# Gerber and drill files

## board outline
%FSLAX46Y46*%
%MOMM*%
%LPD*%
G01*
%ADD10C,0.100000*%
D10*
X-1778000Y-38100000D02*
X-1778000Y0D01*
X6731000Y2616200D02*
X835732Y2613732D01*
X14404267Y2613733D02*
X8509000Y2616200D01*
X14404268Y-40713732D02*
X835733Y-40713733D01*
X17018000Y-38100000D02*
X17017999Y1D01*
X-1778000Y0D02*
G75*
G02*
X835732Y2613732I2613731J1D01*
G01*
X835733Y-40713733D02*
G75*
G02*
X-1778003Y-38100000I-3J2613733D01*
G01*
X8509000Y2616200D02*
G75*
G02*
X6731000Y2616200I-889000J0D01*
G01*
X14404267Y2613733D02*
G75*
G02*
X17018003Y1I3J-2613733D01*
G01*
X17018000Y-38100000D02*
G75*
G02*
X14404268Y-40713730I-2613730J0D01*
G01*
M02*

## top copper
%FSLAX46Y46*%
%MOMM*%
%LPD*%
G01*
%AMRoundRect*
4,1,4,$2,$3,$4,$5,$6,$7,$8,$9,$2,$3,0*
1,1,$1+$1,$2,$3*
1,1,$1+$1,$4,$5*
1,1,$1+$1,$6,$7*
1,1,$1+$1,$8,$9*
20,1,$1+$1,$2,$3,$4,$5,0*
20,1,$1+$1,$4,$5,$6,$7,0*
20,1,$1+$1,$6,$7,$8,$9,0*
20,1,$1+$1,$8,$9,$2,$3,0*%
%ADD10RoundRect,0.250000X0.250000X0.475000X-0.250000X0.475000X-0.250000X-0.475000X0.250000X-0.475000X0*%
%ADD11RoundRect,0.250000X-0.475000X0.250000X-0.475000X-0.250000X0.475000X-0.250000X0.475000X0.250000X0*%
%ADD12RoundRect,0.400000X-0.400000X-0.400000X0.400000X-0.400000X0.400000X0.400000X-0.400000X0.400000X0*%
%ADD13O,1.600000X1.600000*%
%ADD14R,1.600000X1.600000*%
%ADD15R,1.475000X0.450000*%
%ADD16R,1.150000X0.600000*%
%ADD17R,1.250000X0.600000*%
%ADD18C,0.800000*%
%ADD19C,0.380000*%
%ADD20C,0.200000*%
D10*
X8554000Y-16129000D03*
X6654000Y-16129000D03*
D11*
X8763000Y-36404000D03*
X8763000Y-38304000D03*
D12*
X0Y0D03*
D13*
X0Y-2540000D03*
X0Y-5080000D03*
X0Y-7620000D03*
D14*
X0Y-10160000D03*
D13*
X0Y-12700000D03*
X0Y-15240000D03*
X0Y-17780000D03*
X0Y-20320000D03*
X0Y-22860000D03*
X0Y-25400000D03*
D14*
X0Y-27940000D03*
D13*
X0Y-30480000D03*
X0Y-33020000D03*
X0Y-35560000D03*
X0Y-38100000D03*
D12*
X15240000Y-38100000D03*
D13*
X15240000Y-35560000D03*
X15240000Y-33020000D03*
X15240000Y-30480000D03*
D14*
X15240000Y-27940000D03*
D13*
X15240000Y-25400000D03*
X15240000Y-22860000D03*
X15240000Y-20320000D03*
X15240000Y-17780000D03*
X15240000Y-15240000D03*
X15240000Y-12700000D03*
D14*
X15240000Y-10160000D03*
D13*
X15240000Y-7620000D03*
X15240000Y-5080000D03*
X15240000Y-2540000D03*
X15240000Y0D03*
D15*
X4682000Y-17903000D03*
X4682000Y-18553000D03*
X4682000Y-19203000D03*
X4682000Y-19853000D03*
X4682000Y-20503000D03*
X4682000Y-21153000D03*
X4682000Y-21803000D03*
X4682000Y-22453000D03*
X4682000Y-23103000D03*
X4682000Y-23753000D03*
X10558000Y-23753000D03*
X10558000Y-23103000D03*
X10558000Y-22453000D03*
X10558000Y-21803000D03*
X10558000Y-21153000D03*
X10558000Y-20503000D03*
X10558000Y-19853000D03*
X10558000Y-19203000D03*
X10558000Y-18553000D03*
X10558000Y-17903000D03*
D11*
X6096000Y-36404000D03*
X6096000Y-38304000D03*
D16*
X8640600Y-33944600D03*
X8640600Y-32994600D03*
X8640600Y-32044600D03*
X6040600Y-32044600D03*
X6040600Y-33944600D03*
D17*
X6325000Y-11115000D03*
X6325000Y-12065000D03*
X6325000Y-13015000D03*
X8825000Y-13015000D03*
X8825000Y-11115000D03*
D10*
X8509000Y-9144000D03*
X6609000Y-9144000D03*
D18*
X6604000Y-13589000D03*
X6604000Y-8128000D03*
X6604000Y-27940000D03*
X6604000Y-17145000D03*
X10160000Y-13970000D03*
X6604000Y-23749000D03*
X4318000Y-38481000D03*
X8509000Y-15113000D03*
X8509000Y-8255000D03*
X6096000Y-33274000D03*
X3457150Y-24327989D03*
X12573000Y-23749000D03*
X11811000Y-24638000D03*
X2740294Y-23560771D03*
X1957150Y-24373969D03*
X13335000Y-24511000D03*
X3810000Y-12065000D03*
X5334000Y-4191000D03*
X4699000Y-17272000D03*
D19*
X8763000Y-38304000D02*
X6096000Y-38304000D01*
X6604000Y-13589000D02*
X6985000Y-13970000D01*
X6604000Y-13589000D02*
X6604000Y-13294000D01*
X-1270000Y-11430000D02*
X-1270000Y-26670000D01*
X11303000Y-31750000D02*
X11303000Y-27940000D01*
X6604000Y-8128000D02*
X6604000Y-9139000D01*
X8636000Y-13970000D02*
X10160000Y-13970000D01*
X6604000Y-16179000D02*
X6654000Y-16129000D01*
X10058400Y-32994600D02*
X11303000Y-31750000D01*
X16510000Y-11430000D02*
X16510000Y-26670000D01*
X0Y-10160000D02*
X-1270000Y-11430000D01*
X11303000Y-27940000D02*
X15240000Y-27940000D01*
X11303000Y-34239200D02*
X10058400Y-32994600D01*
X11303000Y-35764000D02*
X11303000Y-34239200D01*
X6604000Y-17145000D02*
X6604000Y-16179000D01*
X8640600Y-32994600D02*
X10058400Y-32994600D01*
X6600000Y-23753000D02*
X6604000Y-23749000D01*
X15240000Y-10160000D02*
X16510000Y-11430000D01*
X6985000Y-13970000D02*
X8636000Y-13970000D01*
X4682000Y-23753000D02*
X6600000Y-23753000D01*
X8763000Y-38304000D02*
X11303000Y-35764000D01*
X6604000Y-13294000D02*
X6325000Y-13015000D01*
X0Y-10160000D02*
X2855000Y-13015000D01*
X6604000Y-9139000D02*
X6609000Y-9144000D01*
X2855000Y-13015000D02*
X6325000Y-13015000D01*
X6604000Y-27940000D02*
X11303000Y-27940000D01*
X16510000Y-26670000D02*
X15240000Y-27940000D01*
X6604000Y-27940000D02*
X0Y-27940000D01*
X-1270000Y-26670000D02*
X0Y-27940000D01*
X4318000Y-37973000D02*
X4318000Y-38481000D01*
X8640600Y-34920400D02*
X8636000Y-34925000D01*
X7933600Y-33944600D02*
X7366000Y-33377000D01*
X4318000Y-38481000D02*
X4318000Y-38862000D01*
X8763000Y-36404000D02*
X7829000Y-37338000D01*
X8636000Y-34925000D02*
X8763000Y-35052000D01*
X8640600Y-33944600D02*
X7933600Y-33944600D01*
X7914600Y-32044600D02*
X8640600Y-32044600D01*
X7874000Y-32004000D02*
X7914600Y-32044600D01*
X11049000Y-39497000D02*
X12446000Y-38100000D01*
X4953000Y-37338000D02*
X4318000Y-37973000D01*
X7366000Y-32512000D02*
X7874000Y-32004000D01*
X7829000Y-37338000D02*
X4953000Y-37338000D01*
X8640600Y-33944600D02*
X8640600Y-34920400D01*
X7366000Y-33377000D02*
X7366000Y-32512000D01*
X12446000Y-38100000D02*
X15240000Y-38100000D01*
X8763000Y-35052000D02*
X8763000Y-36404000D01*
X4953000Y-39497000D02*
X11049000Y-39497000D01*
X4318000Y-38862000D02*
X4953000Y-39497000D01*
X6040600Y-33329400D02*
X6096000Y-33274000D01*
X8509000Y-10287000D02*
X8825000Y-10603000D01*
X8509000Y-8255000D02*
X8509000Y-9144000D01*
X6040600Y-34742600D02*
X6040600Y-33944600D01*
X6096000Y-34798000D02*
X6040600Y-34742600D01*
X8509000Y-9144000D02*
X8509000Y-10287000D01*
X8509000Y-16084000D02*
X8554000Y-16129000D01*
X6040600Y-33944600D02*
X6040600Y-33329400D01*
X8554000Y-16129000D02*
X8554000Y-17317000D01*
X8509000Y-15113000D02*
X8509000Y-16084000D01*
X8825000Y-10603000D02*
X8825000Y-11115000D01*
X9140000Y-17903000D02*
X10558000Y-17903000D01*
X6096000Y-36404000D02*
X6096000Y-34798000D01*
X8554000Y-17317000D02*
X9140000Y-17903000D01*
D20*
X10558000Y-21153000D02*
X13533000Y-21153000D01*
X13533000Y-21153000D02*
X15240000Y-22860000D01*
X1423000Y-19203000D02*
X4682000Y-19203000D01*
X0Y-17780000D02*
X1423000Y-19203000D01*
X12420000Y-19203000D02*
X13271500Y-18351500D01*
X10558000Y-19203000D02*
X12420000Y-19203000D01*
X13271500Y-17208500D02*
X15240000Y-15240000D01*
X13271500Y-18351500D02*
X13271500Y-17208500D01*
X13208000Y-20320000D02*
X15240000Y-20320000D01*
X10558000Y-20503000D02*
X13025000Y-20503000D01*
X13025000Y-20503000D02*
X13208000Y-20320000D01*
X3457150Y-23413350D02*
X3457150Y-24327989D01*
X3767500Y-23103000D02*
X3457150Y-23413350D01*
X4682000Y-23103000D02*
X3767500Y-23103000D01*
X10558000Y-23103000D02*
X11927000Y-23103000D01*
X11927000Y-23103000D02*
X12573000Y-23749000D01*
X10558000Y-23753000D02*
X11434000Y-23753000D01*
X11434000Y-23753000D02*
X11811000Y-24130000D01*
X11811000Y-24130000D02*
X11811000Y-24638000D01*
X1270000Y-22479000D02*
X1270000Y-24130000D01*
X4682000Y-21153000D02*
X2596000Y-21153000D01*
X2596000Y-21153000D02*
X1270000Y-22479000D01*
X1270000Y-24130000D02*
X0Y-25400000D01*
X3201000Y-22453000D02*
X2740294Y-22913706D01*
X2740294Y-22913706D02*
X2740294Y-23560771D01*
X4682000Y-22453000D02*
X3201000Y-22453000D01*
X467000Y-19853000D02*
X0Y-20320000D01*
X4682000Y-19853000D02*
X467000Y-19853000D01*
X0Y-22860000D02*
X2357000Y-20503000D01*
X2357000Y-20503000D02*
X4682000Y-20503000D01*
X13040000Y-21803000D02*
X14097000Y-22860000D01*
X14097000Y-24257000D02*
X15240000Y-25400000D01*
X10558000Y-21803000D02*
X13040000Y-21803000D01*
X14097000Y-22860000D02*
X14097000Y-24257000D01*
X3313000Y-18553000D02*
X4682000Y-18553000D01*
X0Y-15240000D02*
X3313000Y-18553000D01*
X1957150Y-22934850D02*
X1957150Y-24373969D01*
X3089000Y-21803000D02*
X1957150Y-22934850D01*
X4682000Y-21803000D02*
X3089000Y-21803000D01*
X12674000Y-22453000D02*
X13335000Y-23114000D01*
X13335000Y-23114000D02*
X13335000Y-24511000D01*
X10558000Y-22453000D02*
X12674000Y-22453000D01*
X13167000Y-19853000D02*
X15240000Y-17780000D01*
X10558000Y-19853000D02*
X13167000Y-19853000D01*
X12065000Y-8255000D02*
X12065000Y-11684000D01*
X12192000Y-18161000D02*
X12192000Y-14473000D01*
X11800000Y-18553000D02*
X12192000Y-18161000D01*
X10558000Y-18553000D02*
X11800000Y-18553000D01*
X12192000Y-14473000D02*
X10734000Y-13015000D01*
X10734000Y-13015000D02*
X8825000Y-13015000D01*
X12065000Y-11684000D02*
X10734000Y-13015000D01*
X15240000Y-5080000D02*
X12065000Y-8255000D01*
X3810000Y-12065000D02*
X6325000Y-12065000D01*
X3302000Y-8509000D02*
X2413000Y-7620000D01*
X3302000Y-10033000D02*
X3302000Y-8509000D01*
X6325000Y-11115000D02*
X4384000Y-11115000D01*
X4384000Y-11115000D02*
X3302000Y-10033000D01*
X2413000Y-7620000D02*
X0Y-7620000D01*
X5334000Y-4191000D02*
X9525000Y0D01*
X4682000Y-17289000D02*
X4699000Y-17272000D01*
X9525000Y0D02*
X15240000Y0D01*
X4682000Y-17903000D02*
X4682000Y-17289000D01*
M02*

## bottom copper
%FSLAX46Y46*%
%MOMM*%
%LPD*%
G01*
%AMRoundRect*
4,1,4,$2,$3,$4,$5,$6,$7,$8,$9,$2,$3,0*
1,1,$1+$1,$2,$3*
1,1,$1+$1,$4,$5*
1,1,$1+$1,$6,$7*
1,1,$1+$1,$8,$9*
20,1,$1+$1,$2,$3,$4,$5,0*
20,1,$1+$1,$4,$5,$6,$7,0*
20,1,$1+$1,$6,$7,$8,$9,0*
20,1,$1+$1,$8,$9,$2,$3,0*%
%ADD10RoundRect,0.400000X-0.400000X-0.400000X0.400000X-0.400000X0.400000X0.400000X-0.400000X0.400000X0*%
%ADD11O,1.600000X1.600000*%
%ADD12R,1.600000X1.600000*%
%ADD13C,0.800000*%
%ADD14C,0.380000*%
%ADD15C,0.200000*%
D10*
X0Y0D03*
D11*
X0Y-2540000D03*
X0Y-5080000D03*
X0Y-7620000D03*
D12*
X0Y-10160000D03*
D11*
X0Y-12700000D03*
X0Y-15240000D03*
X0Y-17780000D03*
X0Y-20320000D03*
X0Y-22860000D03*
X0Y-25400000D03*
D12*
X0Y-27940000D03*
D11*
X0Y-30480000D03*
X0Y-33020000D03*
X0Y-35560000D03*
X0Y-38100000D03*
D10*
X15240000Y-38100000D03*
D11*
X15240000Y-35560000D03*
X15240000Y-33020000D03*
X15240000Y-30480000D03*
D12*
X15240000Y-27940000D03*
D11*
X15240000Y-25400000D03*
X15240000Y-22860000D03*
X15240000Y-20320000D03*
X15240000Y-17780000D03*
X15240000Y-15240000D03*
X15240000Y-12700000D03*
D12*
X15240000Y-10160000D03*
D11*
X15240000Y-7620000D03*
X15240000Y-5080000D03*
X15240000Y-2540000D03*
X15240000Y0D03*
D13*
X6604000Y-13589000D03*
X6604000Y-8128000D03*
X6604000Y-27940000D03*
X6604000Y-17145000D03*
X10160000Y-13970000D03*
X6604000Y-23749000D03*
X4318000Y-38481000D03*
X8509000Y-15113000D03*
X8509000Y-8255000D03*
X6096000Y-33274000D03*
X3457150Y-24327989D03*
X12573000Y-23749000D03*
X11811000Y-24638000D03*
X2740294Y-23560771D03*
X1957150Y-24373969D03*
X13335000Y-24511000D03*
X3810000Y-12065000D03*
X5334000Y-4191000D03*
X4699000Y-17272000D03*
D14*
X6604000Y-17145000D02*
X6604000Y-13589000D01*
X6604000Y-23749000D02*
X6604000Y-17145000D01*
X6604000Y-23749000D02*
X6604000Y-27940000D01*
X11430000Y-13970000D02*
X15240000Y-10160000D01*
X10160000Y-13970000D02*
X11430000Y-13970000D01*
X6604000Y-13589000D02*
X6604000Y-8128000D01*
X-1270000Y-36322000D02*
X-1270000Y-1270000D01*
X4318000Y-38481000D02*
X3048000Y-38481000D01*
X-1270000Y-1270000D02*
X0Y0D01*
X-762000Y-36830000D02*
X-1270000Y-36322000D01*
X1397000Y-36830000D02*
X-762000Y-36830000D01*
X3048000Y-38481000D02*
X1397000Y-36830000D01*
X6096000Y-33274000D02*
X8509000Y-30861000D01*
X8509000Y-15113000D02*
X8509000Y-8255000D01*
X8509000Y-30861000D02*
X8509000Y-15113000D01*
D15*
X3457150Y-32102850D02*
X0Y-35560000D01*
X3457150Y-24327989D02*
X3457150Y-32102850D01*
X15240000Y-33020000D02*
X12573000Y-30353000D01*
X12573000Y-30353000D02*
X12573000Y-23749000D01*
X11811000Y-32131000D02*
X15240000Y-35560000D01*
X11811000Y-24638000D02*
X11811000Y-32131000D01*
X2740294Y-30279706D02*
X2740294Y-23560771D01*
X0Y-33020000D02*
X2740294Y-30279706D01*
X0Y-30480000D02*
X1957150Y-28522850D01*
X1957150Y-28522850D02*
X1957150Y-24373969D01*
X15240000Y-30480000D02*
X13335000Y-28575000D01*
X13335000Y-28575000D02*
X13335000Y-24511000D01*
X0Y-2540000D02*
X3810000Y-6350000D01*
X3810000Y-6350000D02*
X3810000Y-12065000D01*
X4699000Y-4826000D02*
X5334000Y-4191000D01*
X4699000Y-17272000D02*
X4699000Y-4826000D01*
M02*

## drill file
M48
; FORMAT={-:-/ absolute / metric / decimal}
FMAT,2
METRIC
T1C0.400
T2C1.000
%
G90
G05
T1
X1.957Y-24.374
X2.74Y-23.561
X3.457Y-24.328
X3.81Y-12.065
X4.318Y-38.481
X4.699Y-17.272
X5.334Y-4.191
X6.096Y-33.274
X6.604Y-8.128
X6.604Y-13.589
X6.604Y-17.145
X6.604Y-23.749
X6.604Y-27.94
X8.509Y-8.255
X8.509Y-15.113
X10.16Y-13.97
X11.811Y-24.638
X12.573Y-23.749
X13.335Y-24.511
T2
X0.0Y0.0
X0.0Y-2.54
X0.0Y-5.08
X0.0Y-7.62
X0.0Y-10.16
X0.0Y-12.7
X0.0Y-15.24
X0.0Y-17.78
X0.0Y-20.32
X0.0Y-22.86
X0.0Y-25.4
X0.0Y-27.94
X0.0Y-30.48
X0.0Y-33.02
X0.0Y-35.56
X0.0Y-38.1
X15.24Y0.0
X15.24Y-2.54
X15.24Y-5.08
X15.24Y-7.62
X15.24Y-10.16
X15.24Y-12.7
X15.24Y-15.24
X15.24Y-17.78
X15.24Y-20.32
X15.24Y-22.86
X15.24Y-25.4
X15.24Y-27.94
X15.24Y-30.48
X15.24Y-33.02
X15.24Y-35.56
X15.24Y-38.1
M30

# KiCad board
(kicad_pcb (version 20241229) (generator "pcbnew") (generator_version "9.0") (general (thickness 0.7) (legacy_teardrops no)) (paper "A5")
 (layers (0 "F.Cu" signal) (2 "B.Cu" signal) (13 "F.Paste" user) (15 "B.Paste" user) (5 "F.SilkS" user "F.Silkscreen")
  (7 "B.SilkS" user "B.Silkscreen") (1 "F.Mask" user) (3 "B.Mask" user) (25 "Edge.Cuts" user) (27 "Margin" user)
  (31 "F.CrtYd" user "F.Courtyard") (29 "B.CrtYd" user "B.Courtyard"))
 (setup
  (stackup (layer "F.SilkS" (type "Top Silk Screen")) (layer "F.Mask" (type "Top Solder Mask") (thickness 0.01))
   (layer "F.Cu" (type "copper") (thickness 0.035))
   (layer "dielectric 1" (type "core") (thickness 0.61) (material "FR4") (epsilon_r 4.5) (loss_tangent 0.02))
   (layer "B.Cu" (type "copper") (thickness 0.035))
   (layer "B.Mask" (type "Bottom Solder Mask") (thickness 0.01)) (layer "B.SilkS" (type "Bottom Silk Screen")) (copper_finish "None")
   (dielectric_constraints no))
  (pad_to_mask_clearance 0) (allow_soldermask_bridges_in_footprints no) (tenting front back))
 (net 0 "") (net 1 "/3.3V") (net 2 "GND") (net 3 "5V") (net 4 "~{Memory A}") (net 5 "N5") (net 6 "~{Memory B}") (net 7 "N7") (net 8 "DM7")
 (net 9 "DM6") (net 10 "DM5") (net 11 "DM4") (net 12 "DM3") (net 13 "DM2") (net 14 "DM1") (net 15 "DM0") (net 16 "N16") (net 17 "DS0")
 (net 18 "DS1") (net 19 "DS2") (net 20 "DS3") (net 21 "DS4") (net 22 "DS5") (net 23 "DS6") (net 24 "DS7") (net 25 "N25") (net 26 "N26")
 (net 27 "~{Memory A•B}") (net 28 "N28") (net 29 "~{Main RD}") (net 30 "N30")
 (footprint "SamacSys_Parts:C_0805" (layer "F.Cu") (at 7.62 16.129 90)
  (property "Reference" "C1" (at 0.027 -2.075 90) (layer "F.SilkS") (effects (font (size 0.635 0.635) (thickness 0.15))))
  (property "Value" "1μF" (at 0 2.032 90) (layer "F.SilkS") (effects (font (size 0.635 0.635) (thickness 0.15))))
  (pad "1" smd roundrect (at 0 0.934 180) (size 1 1.45) (layers "F.Cu" "F.Mask" "F.Paste") (roundrect_rratio 0.25) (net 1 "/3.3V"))
  (pad "2" smd roundrect (at 0 -0.966 180) (size 1 1.45) (layers "F.Cu" "F.Mask" "F.Paste") (roundrect_rratio 0.25) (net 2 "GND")))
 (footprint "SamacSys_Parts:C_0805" (layer "F.Cu") (at 8.763 37.338 180)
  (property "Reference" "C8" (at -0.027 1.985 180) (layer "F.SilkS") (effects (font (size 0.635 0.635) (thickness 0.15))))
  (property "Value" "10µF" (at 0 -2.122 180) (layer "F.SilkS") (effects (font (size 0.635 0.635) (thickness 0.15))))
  (pad "1" smd roundrect (at 0 0.934 270) (size 1 1.45) (layers "F.Cu" "F.Mask" "F.Paste") (roundrect_rratio 0.25) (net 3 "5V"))
  (pad "2" smd roundrect (at 0 -0.966 270) (size 1 1.45) (layers "F.Cu" "F.Mask" "F.Paste") (roundrect_rratio 0.25) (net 2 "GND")))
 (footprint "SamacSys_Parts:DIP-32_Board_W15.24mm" (layer "F.Cu") (at 0 0)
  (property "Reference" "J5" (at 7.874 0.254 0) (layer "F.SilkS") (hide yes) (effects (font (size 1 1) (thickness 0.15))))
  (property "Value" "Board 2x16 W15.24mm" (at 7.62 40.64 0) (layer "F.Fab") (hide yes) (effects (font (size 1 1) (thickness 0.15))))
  (fp_line (start -1.778 38.1) (end -1.778 0) (stroke (width 0.1) (type solid)) (layer "Edge.Cuts"))
  (fp_line (start 6.731 -2.6162) (end 0.835732 -2.613732) (stroke (width 0.1) (type solid)) (layer "Edge.Cuts"))
  (fp_line (start 14.404267 -2.613733) (end 8.509 -2.6162) (stroke (width 0.1) (type solid)) (layer "Edge.Cuts"))
  (fp_line (start 14.404268 40.713732) (end 0.835733 40.713733) (stroke (width 0.1) (type solid)) (layer "Edge.Cuts"))
  (fp_line (start 17.018 38.1) (end 17.017999 -0.000001) (stroke (width 0.1) (type solid)) (layer "Edge.Cuts"))
  (fp_arc (start -1.778 0) (mid -1.012456 -1.848188) (end 0.835732 -2.613732) (stroke (width 0.1) (type solid)) (layer "Edge.Cuts"))
  (fp_arc (start 0.835733 40.713733) (mid -1.012456 39.948189) (end -1.778 38.1) (stroke (width 0.1) (type solid)) (layer "Edge.Cuts"))
  (fp_arc (start 8.509 -2.6162) (mid 7.62 -1.7272) (end 6.731 -2.6162) (stroke (width 0.1) (type default)) (layer "Edge.Cuts"))
  (fp_arc (start 14.404267 -2.613733) (mid 16.252455 -1.848189) (end 17.017999 -0.000001) (stroke (width 0.1) (type solid))
   (layer "Edge.Cuts"))
  (fp_arc (start 17.018 38.1) (mid 16.252455 39.948187) (end 14.404268 40.713732) (stroke (width 0.1) (type solid)) (layer "Edge.Cuts"))
  (pad "1" thru_hole roundrect (at 0 0) (size 1.6 1.6) (drill 1) (layers "*.Cu" "*.Mask") (remove_unused_layers no) (roundrect_rratio 0.25)
   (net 3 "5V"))
  (pad "2" thru_hole oval (at 0 2.54) (size 1.6 1.6) (drill 1) (layers "*.Cu" "*.Mask") (remove_unused_layers no) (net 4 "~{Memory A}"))
  (pad "3" thru_hole oval (at 0 5.08) (size 1.6 1.6) (drill 1) (layers "*.Cu" "*.Mask") (remove_unused_layers no) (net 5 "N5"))
  (pad "4" thru_hole oval (at 0 7.62) (size 1.6 1.6) (drill 1) (layers "*.Cu" "*.Mask") (remove_unused_layers no) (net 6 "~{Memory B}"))
  (pad "5" thru_hole rect (at 0 10.16) (size 1.6 1.6) (drill 1) (layers "*.Cu" "*.Mask") (remove_unused_layers no) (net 2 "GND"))
  (pad "6" thru_hole oval (at 0 12.7) (size 1.6 1.6) (drill 1) (layers "*.Cu" "*.Mask") (remove_unused_layers no) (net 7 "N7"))
  (pad "7" thru_hole oval (at 0 15.24) (size 1.6 1.6) (drill 1) (layers "*.Cu" "*.Mask") (remove_unused_layers no) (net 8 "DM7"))
  (pad "8" thru_hole oval (at 0 17.78) (size 1.6 1.6) (drill 1) (layers "*.Cu" "*.Mask") (remove_unused_layers no) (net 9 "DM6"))
  (pad "9" thru_hole oval (at 0 20.32) (size 1.6 1.6) (drill 1) (layers "*.Cu" "*.Mask") (remove_unused_layers no) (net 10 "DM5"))
  (pad "10" thru_hole oval (at 0 22.86) (size 1.6 1.6) (drill 1) (layers "*.Cu" "*.Mask") (remove_unused_layers no) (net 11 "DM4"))
  (pad "11" thru_hole oval (at 0 25.4) (size 1.6 1.6) (drill 1) (layers "*.Cu" "*.Mask") (remove_unused_layers no) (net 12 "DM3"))
  (pad "12" thru_hole rect (at 0 27.94) (size 1.6 1.6) (drill 1) (layers "*.Cu" "*.Mask") (remove_unused_layers no) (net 2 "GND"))
  (pad "13" thru_hole oval (at 0 30.48) (size 1.6 1.6) (drill 1) (layers "*.Cu" "*.Mask") (remove_unused_layers no) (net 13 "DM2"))
  (pad "14" thru_hole oval (at 0 33.02) (size 1.6 1.6) (drill 1) (layers "*.Cu" "*.Mask") (remove_unused_layers no) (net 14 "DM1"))
  (pad "15" thru_hole oval (at 0 35.56) (size 1.6 1.6) (drill 1) (layers "*.Cu" "*.Mask") (remove_unused_layers no) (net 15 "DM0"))
  (pad "16" thru_hole oval (at 0 38.1) (size 1.6 1.6) (drill 1) (layers "*.Cu" "*.Mask") (remove_unused_layers no) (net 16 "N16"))
  (pad "17" thru_hole roundrect (at 15.24 38.1) (size 1.6 1.6) (drill 1) (layers "*.Cu" "*.Mask") (remove_unused_layers no)
   (roundrect_rratio 0.25) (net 3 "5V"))
  (pad "18" thru_hole oval (at 15.24 35.56 180) (size 1.6 1.6) (drill 1) (layers "*.Cu" "*.Mask") (remove_unused_layers no) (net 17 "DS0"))
  (pad "19" thru_hole oval (at 15.24 33.02 180) (size 1.6 1.6) (drill 1) (layers "*.Cu" "*.Mask") (remove_unused_layers no) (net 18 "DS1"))
  (pad "20" thru_hole oval (at 15.24 30.48 180) (size 1.6 1.6) (drill 1) (layers "*.Cu" "*.Mask") (remove_unused_layers no) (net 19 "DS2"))
  (pad "21" thru_hole rect (at 15.24 27.94) (size 1.6 1.6) (drill 1) (layers "*.Cu" "*.Mask") (remove_unused_layers no) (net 2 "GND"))
  (pad "22" thru_hole oval (at 15.24 25.4) (size 1.6 1.6) (drill 1) (layers "*.Cu" "*.Mask") (remove_unused_layers no) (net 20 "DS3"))
  (pad "23" thru_hole oval (at 15.24 22.86) (size 1.6 1.6) (drill 1) (layers "*.Cu" "*.Mask") (remove_unused_layers no) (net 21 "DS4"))
  (pad "24" thru_hole oval (at 15.24 20.32) (size 1.6 1.6) (drill 1) (layers "*.Cu" "*.Mask") (remove_unused_layers no) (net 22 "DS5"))
  (pad "25" thru_hole oval (at 15.24 17.78) (size 1.6 1.6) (drill 1) (layers "*.Cu" "*.Mask") (remove_unused_layers no) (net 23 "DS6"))
  (pad "26" thru_hole oval (at 15.24 15.24) (size 1.6 1.6) (drill 1) (layers "*.Cu" "*.Mask") (remove_unused_layers no) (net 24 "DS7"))
  (pad "27" thru_hole oval (at 15.24 12.7) (size 1.6 1.6) (drill 1) (layers "*.Cu" "*.Mask") (remove_unused_layers no) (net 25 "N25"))
  (pad "28" thru_hole rect (at 15.24 10.16) (size 1.6 1.6) (drill 1) (layers "*.Cu" "*.Mask") (remove_unused_layers no) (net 2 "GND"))
  (pad "29" thru_hole oval (at 15.24 7.62) (size 1.6 1.6) (drill 1) (layers "*.Cu" "*.Mask") (remove_unused_layers no) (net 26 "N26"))
  (pad "30" thru_hole oval (at 15.24 5.08) (size 1.6 1.6) (drill 1) (layers "*.Cu" "*.Mask") (remove_unused_layers no)
   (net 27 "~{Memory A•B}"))
  (pad "31" thru_hole oval (at 15.24 2.54) (size 1.6 1.6) (drill 1) (layers "*.Cu" "*.Mask") (remove_unused_layers no) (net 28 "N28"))
  (pad "32" thru_hole oval (at 15.24 0) (size 1.6 1.6) (drill 1) (layers "*.Cu" "*.Mask") (remove_unused_layers no) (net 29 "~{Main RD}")))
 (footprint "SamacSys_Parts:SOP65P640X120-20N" (layer "F.Cu") (at 7.62 20.828)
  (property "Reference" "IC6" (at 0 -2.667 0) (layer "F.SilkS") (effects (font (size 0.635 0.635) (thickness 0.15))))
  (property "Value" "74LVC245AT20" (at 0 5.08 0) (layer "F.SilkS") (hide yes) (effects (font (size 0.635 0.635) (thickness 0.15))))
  (pad "1" smd rect (at -2.938 -2.925 90) (size 0.45 1.475) (layers "F.Cu" "F.Mask" "F.Paste") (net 29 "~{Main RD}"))
  (pad "2" smd rect (at -2.938 -2.275 90) (size 0.45 1.475) (layers "F.Cu" "F.Mask" "F.Paste") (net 8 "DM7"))
  (pad "3" smd rect (at -2.938 -1.625 90) (size 0.45 1.475) (layers "F.Cu" "F.Mask" "F.Paste") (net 9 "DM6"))
  (pad "4" smd rect (at -2.938 -0.975 90) (size 0.45 1.475) (layers "F.Cu" "F.Mask" "F.Paste") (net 10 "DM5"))
  (pad "5" smd rect (at -2.938 -0.325 90) (size 0.45 1.475) (layers "F.Cu" "F.Mask" "F.Paste") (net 11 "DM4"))
  (pad "6" smd rect (at -2.938 0.325 90) (size 0.45 1.475) (layers "F.Cu" "F.Mask" "F.Paste") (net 12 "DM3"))
  (pad "7" smd rect (at -2.938 0.975 90) (size 0.45 1.475) (layers "F.Cu" "F.Mask" "F.Paste") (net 13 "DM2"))
  (pad "8" smd rect (at -2.938 1.625 90) (size 0.45 1.475) (layers "F.Cu" "F.Mask" "F.Paste") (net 14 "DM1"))
  (pad "9" smd rect (at -2.938 2.275 90) (size 0.45 1.475) (layers "F.Cu" "F.Mask" "F.Paste") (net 15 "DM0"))
  (pad "10" smd rect (at -2.938 2.925 90) (size 0.45 1.475) (layers "F.Cu" "F.Mask" "F.Paste") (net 2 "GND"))
  (pad "11" smd rect (at 2.938 2.925 90) (size 0.45 1.475) (layers "F.Cu" "F.Mask" "F.Paste") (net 17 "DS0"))
  (pad "12" smd rect (at 2.938 2.275 90) (size 0.45 1.475) (layers "F.Cu" "F.Mask" "F.Paste") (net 18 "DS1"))
  (pad "13" smd rect (at 2.938 1.625 90) (size 0.45 1.475) (layers "F.Cu" "F.Mask" "F.Paste") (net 19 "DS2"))
  (pad "14" smd rect (at 2.938 0.975 90) (size 0.45 1.475) (layers "F.Cu" "F.Mask" "F.Paste") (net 20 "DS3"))
  (pad "15" smd rect (at 2.938 0.325 90) (size 0.45 1.475) (layers "F.Cu" "F.Mask" "F.Paste") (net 21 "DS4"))
  (pad "16" smd rect (at 2.938 -0.325 90) (size 0.45 1.475) (layers "F.Cu" "F.Mask" "F.Paste") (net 22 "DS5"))
  (pad "17" smd rect (at 2.938 -0.975 90) (size 0.45 1.475) (layers "F.Cu" "F.Mask" "F.Paste") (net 23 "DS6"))
  (pad "18" smd rect (at 2.938 -1.625 90) (size 0.45 1.475) (layers "F.Cu" "F.Mask" "F.Paste") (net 24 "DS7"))
  (pad "19" smd rect (at 2.938 -2.275 90) (size 0.45 1.475) (layers "F.Cu" "F.Mask" "F.Paste") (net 27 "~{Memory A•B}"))
  (pad "20" smd rect (at 2.938 -2.925 90) (size 0.45 1.475) (layers "F.Cu" "F.Mask" "F.Paste") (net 1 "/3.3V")))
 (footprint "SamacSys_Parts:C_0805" (layer "F.Cu") (at 6.096 37.338 180)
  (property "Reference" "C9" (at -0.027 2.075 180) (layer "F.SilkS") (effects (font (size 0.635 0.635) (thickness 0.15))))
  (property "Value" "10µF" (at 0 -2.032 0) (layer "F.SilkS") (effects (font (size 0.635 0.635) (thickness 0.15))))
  (pad "1" smd roundrect (at 0 0.934 270) (size 1 1.45) (layers "F.Cu" "F.Mask" "F.Paste") (roundrect_rratio 0.25) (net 1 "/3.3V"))
  (pad "2" smd roundrect (at 0 -0.966 270) (size 1 1.45) (layers "F.Cu" "F.Mask" "F.Paste") (roundrect_rratio 0.25) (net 2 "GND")))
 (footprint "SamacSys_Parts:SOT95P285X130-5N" (layer "F.Cu") (at 7.3406 32.9946 180)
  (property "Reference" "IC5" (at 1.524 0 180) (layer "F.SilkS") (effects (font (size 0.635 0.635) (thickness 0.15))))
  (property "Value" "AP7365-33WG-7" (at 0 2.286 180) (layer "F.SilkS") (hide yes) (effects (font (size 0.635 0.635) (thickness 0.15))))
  (pad "1" smd rect (at -1.3 -0.95 270) (size 0.6 1.15) (layers "F.Cu" "F.Mask" "F.Paste") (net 3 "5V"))
  (pad "2" smd rect (at -1.3 0 270) (size 0.6 1.15) (layers "F.Cu" "F.Mask" "F.Paste") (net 2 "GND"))
  (pad "3" smd rect (at -1.3 0.95 270) (size 0.6 1.15) (layers "F.Cu" "F.Mask" "F.Paste") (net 3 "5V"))
  (pad "4" smd rect (at 1.3 0.95 270) (size 0.6 1.15) (layers "F.Cu" "F.Mask" "F.Paste") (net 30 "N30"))
  (pad "5" smd rect (at 1.3 -0.95 270) (size 0.6 1.15) (layers "F.Cu" "F.Mask" "F.Paste") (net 1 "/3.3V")))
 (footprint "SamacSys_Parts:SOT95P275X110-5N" (layer "F.Cu") (at 7.575 12.065)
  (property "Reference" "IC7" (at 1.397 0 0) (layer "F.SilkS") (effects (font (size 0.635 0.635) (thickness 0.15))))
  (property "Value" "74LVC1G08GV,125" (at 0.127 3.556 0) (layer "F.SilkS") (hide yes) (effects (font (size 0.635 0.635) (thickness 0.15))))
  (pad "1" smd rect (at -1.25 -0.95 90) (size 0.6 1.25) (layers "F.Cu" "F.Mask" "F.Paste") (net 6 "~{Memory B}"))
  (pad "2" smd rect (at -1.25 0 90) (size 0.6 1.25) (layers "F.Cu" "F.Mask" "F.Paste") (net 4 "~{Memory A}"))
  (pad "3" smd rect (at -1.25 0.95 90) (size 0.6 1.25) (layers "F.Cu" "F.Mask" "F.Paste") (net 2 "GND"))
  (pad "4" smd rect (at 1.25 0.95 90) (size 0.6 1.25) (layers "F.Cu" "F.Mask" "F.Paste") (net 27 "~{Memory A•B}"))
  (pad "5" smd rect (at 1.25 -0.95 90) (size 0.6 1.25) (layers "F.Cu" "F.Mask" "F.Paste") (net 1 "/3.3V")))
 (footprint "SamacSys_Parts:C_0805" (layer "F.Cu") (at 7.575 9.144 90)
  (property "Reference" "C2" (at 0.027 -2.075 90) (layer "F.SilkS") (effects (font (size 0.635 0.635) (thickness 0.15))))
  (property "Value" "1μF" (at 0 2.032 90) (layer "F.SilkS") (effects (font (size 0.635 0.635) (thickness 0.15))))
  (pad "1" smd roundrect (at 0 0.934 180) (size 1 1.45) (layers "F.Cu" "F.Mask" "F.Paste") (roundrect_rratio 0.25) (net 1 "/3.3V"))
  (pad "2" smd roundrect (at 0 -0.966 180) (size 1 1.45) (layers "F.Cu" "F.Mask" "F.Paste") (roundrect_rratio 0.25) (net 2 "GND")))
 (segment (start 8.763 38.304) (end 6.096 38.304) (width 0.38) (layer "F.Cu") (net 2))
 (segment (start 6.604 13.589) (end 6.985 13.97) (width 0.38) (layer "F.Cu") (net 2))
 (segment (start 6.604 13.589) (end 6.604 13.294) (width 0.38) (layer "F.Cu") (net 2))
 (segment (start -1.27 11.43) (end -1.27 26.67) (width 0.38) (layer "F.Cu") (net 2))
 (segment (start 11.303 31.75) (end 11.303 27.94) (width 0.38) (layer "F.Cu") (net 2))
 (segment (start 6.604 8.128) (end 6.604 9.139) (width 0.38) (layer "F.Cu") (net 2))
 (segment (start 8.636 13.97) (end 10.16 13.97) (width 0.38) (layer "F.Cu") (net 2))
 (segment (start 6.604 16.179) (end 6.654 16.129) (width 0.38) (layer "F.Cu") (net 2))
 (segment (start 10.0584 32.9946) (end 11.303 31.75) (width 0.38) (layer "F.Cu") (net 2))
 (segment (start 16.51 11.43) (end 16.51 26.67) (width 0.38) (layer "F.Cu") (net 2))
 (segment (start 0 10.16) (end -1.27 11.43) (width 0.38) (layer "F.Cu") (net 2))
 (segment (start 11.303 27.94) (end 15.24 27.94) (width 0.38) (layer "F.Cu") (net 2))
 (segment (start 11.303 34.2392) (end 10.0584 32.9946) (width 0.38) (layer "F.Cu") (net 2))
 (segment (start 11.303 35.764) (end 11.303 34.2392) (width 0.38) (layer "F.Cu") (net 2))
 (segment (start 6.604 17.145) (end 6.604 16.179) (width 0.38) (layer "F.Cu") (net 2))
 (segment (start 8.6406 32.9946) (end 10.0584 32.9946) (width 0.38) (layer "F.Cu") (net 2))
 (segment (start 6.6 23.753) (end 6.604 23.749) (width 0.38) (layer "F.Cu") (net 2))
 (segment (start 15.24 10.16) (end 16.51 11.43) (width 0.38) (layer "F.Cu") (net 2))
 (segment (start 6.985 13.97) (end 8.636 13.97) (width 0.38) (layer "F.Cu") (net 2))
 (segment (start 4.682 23.753) (end 6.6 23.753) (width 0.38) (layer "F.Cu") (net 2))
 (segment (start 8.763 38.304) (end 11.303 35.764) (width 0.38) (layer "F.Cu") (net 2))
 (segment (start 6.604 13.294) (end 6.325 13.015) (width 0.38) (layer "F.Cu") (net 2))
 (segment (start 0 10.16) (end 2.855 13.015) (width 0.38) (layer "F.Cu") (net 2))
 (segment (start 6.604 9.139) (end 6.609 9.144) (width 0.38) (layer "F.Cu") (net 2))
 (segment (start 2.855 13.015) (end 6.325 13.015) (width 0.38) (layer "F.Cu") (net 2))
 (segment (start 6.604 27.94) (end 11.303 27.94) (width 0.38) (layer "F.Cu") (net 2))
 (segment (start 16.51 26.67) (end 15.24 27.94) (width 0.38) (layer "F.Cu") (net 2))
 (segment (start 6.604 27.94) (end 0 27.94) (width 0.38) (layer "F.Cu") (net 2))
 (segment (start -1.27 26.67) (end 0 27.94) (width 0.38) (layer "F.Cu") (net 2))
 (via (at 6.604 13.589) (size 0.8) (drill 0.4) (layers "F.Cu" "B.Cu") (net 2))
 (via (at 6.604 8.128) (size 0.8) (drill 0.4) (layers "F.Cu" "B.Cu") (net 2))
 (via (at 6.604 27.94) (size 0.8) (drill 0.4) (layers "F.Cu" "B.Cu") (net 2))
 (via (at 6.604 17.145) (size 0.8) (drill 0.4) (layers "F.Cu" "B.Cu") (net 2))
 (via (at 10.16 13.97) (size 0.8) (drill 0.4) (layers "F.Cu" "B.Cu") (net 2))
 (via (at 6.604 23.749) (size 0.8) (drill 0.4) (layers "F.Cu" "B.Cu") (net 2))
 (segment (start 6.604 17.145) (end 6.604 13.589) (width 0.38) (layer "B.Cu") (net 2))
 (segment (start 6.604 23.749) (end 6.604 17.145) (width 0.38) (layer "B.Cu") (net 2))
 (segment (start 6.604 23.749) (end 6.604 27.94) (width 0.38) (layer "B.Cu") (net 2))
 (segment (start 11.43 13.97) (end 15.24 10.16) (width 0.38) (layer "B.Cu") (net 2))
 (segment (start 10.16 13.97) (end 11.43 13.97) (width 0.38) (layer "B.Cu") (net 2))
 (segment (start 6.604 13.589) (end 6.604 8.128) (width 0.38) (layer "B.Cu") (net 2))
 (segment (start 4.318 37.973) (end 4.318 38.481) (width 0.38) (layer "F.Cu") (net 3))
 (segment (start 8.6406 34.9204) (end 8.636 34.925) (width 0.38) (layer "F.Cu") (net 3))
 (segment (start 7.9336 33.9446) (end 7.366 33.377) (width 0.38) (layer "F.Cu") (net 3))
 (segment (start 4.318 38.481) (end 4.318 38.862) (width 0.38) (layer "F.Cu") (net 3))
 (segment (start 8.763 36.404) (end 7.829 37.338) (width 0.38) (layer "F.Cu") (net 3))
 (segment (start 8.636 34.925) (end 8.763 35.052) (width 0.38) (layer "F.Cu") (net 3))
 (segment (start 8.6406 33.9446) (end 7.9336 33.9446) (width 0.38) (layer "F.Cu") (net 3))
 (segment (start 7.9146 32.0446) (end 8.6406 32.0446) (width 0.38) (layer "F.Cu") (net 3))
 (segment (start 7.874 32.004) (end 7.9146 32.0446) (width 0.38) (layer "F.Cu") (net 3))
 (segment (start 11.049 39.497) (end 12.446 38.1) (width 0.38) (layer "F.Cu") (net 3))
 (segment (start 4.953 37.338) (end 4.318 37.973) (width 0.38) (layer "F.Cu") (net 3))
 (segment (start 7.366 32.512) (end 7.874 32.004) (width 0.38) (layer "F.Cu") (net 3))
 (segment (start 7.829 37.338) (end 4.953 37.338) (width 0.38) (layer "F.Cu") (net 3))
 (segment (start 8.6406 33.9446) (end 8.6406 34.9204) (width 0.38) (layer "F.Cu") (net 3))
 (segment (start 7.366 33.377) (end 7.366 32.512) (width 0.38) (layer "F.Cu") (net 3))
 (segment (start 12.446 38.1) (end 15.24 38.1) (width 0.38) (layer "F.Cu") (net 3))
 (segment (start 8.763 35.052) (end 8.763 36.404) (width 0.38) (layer "F.Cu") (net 3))
 (segment (start 4.953 39.497) (end 11.049 39.497) (width 0.38) (layer "F.Cu") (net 3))
 (segment (start 4.318 38.862) (end 4.953 39.497) (width 0.38) (layer "F.Cu") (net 3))
 (via (at 4.318 38.481) (size 0.8) (drill 0.4) (layers "F.Cu" "B.Cu") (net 3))
 (segment (start -1.27 36.322) (end -1.27 1.27) (width 0.38) (layer "B.Cu") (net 3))
 (segment (start 4.318 38.481) (end 3.048 38.481) (width 0.38) (layer "B.Cu") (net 3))
 (segment (start -1.27 1.27) (end 0 0) (width 0.38) (layer "B.Cu") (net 3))
 (segment (start -0.762 36.83) (end -1.27 36.322) (width 0.38) (layer "B.Cu") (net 3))
 (segment (start 1.397 36.83) (end -0.762 36.83) (width 0.38) (layer "B.Cu") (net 3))
 (segment (start 3.048 38.481) (end 1.397 36.83) (width 0.38) (layer "B.Cu") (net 3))
 (segment (start 6.0406 33.3294) (end 6.096 33.274) (width 0.38) (layer "F.Cu") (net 1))
 (segment (start 8.509 10.287) (end 8.825 10.603) (width 0.38) (layer "F.Cu") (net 1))
 (segment (start 8.509 8.255) (end 8.509 9.144) (width 0.38) (layer "F.Cu") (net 1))
 (segment (start 6.0406 34.7426) (end 6.0406 33.9446) (width 0.38) (layer "F.Cu") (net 1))
 (segment (start 6.096 34.798) (end 6.0406 34.7426) (width 0.38) (layer "F.Cu") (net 1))
 (segment (start 8.509 9.144) (end 8.509 10.287) (width 0.38) (layer "F.Cu") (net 1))
 (segment (start 8.509 16.084) (end 8.554 16.129) (width 0.38) (layer "F.Cu") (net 1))
 (segment (start 6.0406 33.9446) (end 6.0406 33.3294) (width 0.38) (layer "F.Cu") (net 1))
 (segment (start 8.554 16.129) (end 8.554 17.317) (width 0.38) (layer "F.Cu") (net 1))
 (segment (start 8.509 15.113) (end 8.509 16.084) (width 0.38) (layer "F.Cu") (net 1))
 (segment (start 8.825 10.603) (end 8.825 11.115) (width 0.38) (layer "F.Cu") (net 1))
 (segment (start 9.14 17.903) (end 10.558 17.903) (width 0.38) (layer "F.Cu") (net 1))
 (segment (start 6.096 36.404) (end 6.096 34.798) (width 0.38) (layer "F.Cu") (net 1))
 (segment (start 8.554 17.317) (end 9.14 17.903) (width 0.38) (layer "F.Cu") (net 1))
 (via (at 8.509 15.113) (size 0.8) (drill 0.4) (layers "F.Cu" "B.Cu") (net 1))
 (via (at 8.509 8.255) (size 0.8) (drill 0.4) (layers "F.Cu" "B.Cu") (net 1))
 (via (at 6.096 33.274) (size 0.8) (drill 0.4) (layers "F.Cu" "B.Cu") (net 1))
 (segment (start 6.096 33.274) (end 8.509 30.861) (width 0.38) (layer "B.Cu") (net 1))
 (segment (start 8.509 15.113) (end 8.509 8.255) (width 0.38) (layer "B.Cu") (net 1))
 (segment (start 8.509 30.861) (end 8.509 15.113) (width 0.38) (layer "B.Cu") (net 1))
 (segment (start 10.558 21.153) (end 13.533 21.153) (width 0.2) (layer "F.Cu") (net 21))
 (segment (start 13.533 21.153) (end 15.24 22.86) (width 0.2) (layer "F.Cu") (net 21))
 (segment (start 1.423 19.203) (end 4.682 19.203) (width 0.2) (layer "F.Cu") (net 9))
 (segment (start 0 17.78) (end 1.423 19.203) (width 0.2) (layer "F.Cu") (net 9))
 (segment (start 12.42 19.203) (end 13.2715 18.3515) (width 0.2) (layer "F.Cu") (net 24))
 (segment (start 10.558 19.203) (end 12.42 19.203) (width 0.2) (layer "F.Cu") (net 24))
 (segment (start 13.2715 17.2085) (end 15.24 15.24) (width 0.2) (layer "F.Cu") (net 24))
 (segment (start 13.2715 18.3515) (end 13.2715 17.2085) (width 0.2) (layer "F.Cu") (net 24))
 (segment (start 13.208 20.32) (end 15.24 20.32) (width 0.2) (layer "F.Cu") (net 22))
 (segment (start 10.558 20.503) (end 13.025 20.503) (width 0.2) (layer "F.Cu") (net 22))
 (segment (start 13.025 20.503) (end 13.208 20.32) (width 0.2) (layer "F.Cu") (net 22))
 (segment (start 3.45715 23.41335) (end 3.45715 24.327989) (width 0.2) (layer "F.Cu") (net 15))
 (segment (start 3.7675 23.103) (end 3.45715 23.41335) (width 0.2) (layer "F.Cu") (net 15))
 (segment (start 4.682 23.103) (end 3.7675 23.103) (width 0.2) (layer "F.Cu") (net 15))
 (via (at 3.45715 24.327989) (size 0.8) (drill 0.4) (layers "F.Cu" "B.Cu") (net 15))
 (segment (start 3.45715 32.10285) (end 0 35.56) (width 0.2) (layer "B.Cu") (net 15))
 (segment (start 3.45715 24.327989) (end 3.45715 32.10285) (width 0.2) (layer "B.Cu") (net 15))
 (segment (start 10.558 23.103) (end 11.927 23.103) (width 0.2) (layer "F.Cu") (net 18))
 (segment (start 11.927 23.103) (end 12.573 23.749) (width 0.2) (layer "F.Cu") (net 18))
 (via (at 12.573 23.749) (size 0.8) (drill 0.4) (layers "F.Cu" "B.Cu") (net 18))
 (segment (start 15.24 33.02) (end 12.573 30.353) (width 0.2) (layer "B.Cu") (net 18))
 (segment (start 12.573 30.353) (end 12.573 23.749) (width 0.2) (layer "B.Cu") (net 18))
 (segment (start 10.558 23.753) (end 11.434 23.753) (width 0.2) (layer "F.Cu") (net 17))
 (segment (start 11.434 23.753) (end 11.811 24.13) (width 0.2) (layer "F.Cu") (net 17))
 (segment (start 11.811 24.13) (end 11.811 24.638) (width 0.2) (layer "F.Cu") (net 17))
 (via (at 11.811 24.638) (size 0.8) (drill 0.4) (layers "F.Cu" "B.Cu") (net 17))
 (segment (start 11.811 32.131) (end 15.24 35.56) (width 0.2) (layer "B.Cu") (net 17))
 (segment (start 11.811 24.638) (end 11.811 32.131) (width 0.2) (layer "B.Cu") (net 17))
 (segment (start 1.27 22.479) (end 1.27 24.13) (width 0.2) (layer "F.Cu") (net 12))
 (segment (start 4.682 21.153) (end 2.596 21.153) (width 0.2) (layer "F.Cu") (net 12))
 (segment (start 2.596 21.153) (end 1.27 22.479) (width 0.2) (layer "F.Cu") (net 12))
 (segment (start 1.27 24.13) (end 0 25.4) (width 0.2) (layer "F.Cu") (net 12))
 (segment (start 3.201 22.453) (end 2.740294 22.913706) (width 0.2) (layer "F.Cu") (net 14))
 (segment (start 2.740294 22.913706) (end 2.740294 23.560771) (width 0.2) (layer "F.Cu") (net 14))
 (segment (start 4.682 22.453) (end 3.201 22.453) (width 0.2) (layer "F.Cu") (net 14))
 (via (at 2.740294 23.560771) (size 0.8) (drill 0.4) (layers "F.Cu" "B.Cu") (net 14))
 (segment (start 2.740294 30.279706) (end 2.740294 23.560771) (width 0.2) (layer "B.Cu") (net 14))
 (segment (start 0 33.02) (end 2.740294 30.279706) (width 0.2) (layer "B.Cu") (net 14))
 (segment (start 0.467 19.853) (end 0 20.32) (width 0.2) (layer "F.Cu") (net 10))
 (segment (start 4.682 19.853) (end 0.467 19.853) (width 0.2) (layer "F.Cu") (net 10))
 (segment (start 0 22.86) (end 2.357 20.503) (width 0.2) (layer "F.Cu") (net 11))
 (segment (start 2.357 20.503) (end 4.682 20.503) (width 0.2) (layer "F.Cu") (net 11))
 (segment (start 13.04 21.803) (end 14.097 22.86) (width 0.2) (layer "F.Cu") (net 20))
 (segment (start 14.097 24.257) (end 15.24 25.4) (width 0.2) (layer "F.Cu") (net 20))
 (segment (start 10.558 21.803) (end 13.04 21.803) (width 0.2) (layer "F.Cu") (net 20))
 (segment (start 14.097 22.86) (end 14.097 24.257) (width 0.2) (layer "F.Cu") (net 20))
 (segment (start 3.313 18.553) (end 4.682 18.553) (width 0.2) (layer "F.Cu") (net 8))
 (segment (start 0 15.24) (end 3.313 18.553) (width 0.2) (layer "F.Cu") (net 8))
 (segment (start 1.95715 22.93485) (end 1.95715 24.373969) (width 0.2) (layer "F.Cu") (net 13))
 (segment (start 3.089 21.803) (end 1.95715 22.93485) (width 0.2) (layer "F.Cu") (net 13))
 (segment (start 4.682 21.803) (end 3.089 21.803) (width 0.2) (layer "F.Cu") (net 13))
 (via (at 1.95715 24.373969) (size 0.8) (drill 0.4) (layers "F.Cu" "B.Cu") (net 13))
 (segment (start 0 30.48) (end 1.95715 28.52285) (width 0.2) (layer "B.Cu") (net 13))
 (segment (start 1.95715 28.52285) (end 1.95715 24.373969) (width 0.2) (layer "B.Cu") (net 13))
 (segment (start 12.674 22.453) (end 13.335 23.114) (width 0.2) (layer "F.Cu") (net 19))
 (segment (start 13.335 23.114) (end 13.335 24.511) (width 0.2) (layer "F.Cu") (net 19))
 (segment (start 10.558 22.453) (end 12.674 22.453) (width 0.2) (layer "F.Cu") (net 19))
 (via (at 13.335 24.511) (size 0.8) (drill 0.4) (layers "F.Cu" "B.Cu") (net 19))
 (segment (start 15.24 30.48) (end 13.335 28.575) (width 0.2) (layer "B.Cu") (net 19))
 (segment (start 13.335 28.575) (end 13.335 24.511) (width 0.2) (layer "B.Cu") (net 19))
 (segment (start 13.167 19.853) (end 15.24 17.78) (width 0.2) (layer "F.Cu") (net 23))
 (segment (start 10.558 19.853) (end 13.167 19.853) (width 0.2) (layer "F.Cu") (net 23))
 (segment (start 12.065 8.255) (end 12.065 11.684) (width 0.2) (layer "F.Cu") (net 27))
 (segment (start 12.192 18.161) (end 12.192 14.473) (width 0.2) (layer "F.Cu") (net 27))
 (segment (start 11.8 18.553) (end 12.192 18.161) (width 0.2) (layer "F.Cu") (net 27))
 (segment (start 10.558 18.553) (end 11.8 18.553) (width 0.2) (layer "F.Cu") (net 27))
 (segment (start 12.192 14.473) (end 10.734 13.015) (width 0.2) (layer "F.Cu") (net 27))
 (segment (start 10.734 13.015) (end 8.825 13.015) (width 0.2) (layer "F.Cu") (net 27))
 (segment (start 12.065 11.684) (end 10.734 13.015) (width 0.2) (layer "F.Cu") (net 27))
 (segment (start 15.24 5.08) (end 12.065 8.255) (width 0.2) (layer "F.Cu") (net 27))
 (segment (start 3.81 12.065) (end 6.325 12.065) (width 0.2) (layer "F.Cu") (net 4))
 (via (at 3.81 12.065) (size 0.8) (drill 0.4) (layers "F.Cu" "B.Cu") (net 4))
 (segment (start 0 2.54) (end 3.81 6.35) (width 0.2) (layer "B.Cu") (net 4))
 (segment (start 3.81 6.35) (end 3.81 12.065) (width 0.2) (layer "B.Cu") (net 4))
 (segment (start 3.302 8.509) (end 2.413 7.62) (width 0.2) (layer "F.Cu") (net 6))
 (segment (start 3.302 10.033) (end 3.302 8.509) (width 0.2) (layer "F.Cu") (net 6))
 (segment (start 6.325 11.115) (end 4.384 11.115) (width 0.2) (layer "F.Cu") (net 6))
 (segment (start 4.384 11.115) (end 3.302 10.033) (width 0.2) (layer "F.Cu") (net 6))
 (segment (start 2.413 7.62) (end 0 7.62) (width 0.2) (layer "F.Cu") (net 6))
 (segment (start 5.334 4.191) (end 9.525 0) (width 0.2) (layer "F.Cu") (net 29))
 (segment (start 4.682 17.289) (end 4.699 17.272) (width 0.2) (layer "F.Cu") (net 29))
 (segment (start 9.525 0) (end 15.24 0) (width 0.2) (layer "F.Cu") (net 29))
 (segment (start 4.682 17.903) (end 4.682 17.289) (width 0.2) (layer "F.Cu") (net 29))
 (via (at 5.334 4.191) (size 0.8) (drill 0.4) (layers "F.Cu" "B.Cu") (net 29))
 (via (at 4.699 17.272) (size 0.8) (drill 0.4) (layers "F.Cu" "B.Cu") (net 29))
 (segment (start 4.699 4.826) (end 5.334 4.191) (width 0.2) (layer "B.Cu") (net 29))
 (segment (start 4.699 17.272) (end 4.699 4.826) (width 0.2) (layer "B.Cu") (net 29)))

